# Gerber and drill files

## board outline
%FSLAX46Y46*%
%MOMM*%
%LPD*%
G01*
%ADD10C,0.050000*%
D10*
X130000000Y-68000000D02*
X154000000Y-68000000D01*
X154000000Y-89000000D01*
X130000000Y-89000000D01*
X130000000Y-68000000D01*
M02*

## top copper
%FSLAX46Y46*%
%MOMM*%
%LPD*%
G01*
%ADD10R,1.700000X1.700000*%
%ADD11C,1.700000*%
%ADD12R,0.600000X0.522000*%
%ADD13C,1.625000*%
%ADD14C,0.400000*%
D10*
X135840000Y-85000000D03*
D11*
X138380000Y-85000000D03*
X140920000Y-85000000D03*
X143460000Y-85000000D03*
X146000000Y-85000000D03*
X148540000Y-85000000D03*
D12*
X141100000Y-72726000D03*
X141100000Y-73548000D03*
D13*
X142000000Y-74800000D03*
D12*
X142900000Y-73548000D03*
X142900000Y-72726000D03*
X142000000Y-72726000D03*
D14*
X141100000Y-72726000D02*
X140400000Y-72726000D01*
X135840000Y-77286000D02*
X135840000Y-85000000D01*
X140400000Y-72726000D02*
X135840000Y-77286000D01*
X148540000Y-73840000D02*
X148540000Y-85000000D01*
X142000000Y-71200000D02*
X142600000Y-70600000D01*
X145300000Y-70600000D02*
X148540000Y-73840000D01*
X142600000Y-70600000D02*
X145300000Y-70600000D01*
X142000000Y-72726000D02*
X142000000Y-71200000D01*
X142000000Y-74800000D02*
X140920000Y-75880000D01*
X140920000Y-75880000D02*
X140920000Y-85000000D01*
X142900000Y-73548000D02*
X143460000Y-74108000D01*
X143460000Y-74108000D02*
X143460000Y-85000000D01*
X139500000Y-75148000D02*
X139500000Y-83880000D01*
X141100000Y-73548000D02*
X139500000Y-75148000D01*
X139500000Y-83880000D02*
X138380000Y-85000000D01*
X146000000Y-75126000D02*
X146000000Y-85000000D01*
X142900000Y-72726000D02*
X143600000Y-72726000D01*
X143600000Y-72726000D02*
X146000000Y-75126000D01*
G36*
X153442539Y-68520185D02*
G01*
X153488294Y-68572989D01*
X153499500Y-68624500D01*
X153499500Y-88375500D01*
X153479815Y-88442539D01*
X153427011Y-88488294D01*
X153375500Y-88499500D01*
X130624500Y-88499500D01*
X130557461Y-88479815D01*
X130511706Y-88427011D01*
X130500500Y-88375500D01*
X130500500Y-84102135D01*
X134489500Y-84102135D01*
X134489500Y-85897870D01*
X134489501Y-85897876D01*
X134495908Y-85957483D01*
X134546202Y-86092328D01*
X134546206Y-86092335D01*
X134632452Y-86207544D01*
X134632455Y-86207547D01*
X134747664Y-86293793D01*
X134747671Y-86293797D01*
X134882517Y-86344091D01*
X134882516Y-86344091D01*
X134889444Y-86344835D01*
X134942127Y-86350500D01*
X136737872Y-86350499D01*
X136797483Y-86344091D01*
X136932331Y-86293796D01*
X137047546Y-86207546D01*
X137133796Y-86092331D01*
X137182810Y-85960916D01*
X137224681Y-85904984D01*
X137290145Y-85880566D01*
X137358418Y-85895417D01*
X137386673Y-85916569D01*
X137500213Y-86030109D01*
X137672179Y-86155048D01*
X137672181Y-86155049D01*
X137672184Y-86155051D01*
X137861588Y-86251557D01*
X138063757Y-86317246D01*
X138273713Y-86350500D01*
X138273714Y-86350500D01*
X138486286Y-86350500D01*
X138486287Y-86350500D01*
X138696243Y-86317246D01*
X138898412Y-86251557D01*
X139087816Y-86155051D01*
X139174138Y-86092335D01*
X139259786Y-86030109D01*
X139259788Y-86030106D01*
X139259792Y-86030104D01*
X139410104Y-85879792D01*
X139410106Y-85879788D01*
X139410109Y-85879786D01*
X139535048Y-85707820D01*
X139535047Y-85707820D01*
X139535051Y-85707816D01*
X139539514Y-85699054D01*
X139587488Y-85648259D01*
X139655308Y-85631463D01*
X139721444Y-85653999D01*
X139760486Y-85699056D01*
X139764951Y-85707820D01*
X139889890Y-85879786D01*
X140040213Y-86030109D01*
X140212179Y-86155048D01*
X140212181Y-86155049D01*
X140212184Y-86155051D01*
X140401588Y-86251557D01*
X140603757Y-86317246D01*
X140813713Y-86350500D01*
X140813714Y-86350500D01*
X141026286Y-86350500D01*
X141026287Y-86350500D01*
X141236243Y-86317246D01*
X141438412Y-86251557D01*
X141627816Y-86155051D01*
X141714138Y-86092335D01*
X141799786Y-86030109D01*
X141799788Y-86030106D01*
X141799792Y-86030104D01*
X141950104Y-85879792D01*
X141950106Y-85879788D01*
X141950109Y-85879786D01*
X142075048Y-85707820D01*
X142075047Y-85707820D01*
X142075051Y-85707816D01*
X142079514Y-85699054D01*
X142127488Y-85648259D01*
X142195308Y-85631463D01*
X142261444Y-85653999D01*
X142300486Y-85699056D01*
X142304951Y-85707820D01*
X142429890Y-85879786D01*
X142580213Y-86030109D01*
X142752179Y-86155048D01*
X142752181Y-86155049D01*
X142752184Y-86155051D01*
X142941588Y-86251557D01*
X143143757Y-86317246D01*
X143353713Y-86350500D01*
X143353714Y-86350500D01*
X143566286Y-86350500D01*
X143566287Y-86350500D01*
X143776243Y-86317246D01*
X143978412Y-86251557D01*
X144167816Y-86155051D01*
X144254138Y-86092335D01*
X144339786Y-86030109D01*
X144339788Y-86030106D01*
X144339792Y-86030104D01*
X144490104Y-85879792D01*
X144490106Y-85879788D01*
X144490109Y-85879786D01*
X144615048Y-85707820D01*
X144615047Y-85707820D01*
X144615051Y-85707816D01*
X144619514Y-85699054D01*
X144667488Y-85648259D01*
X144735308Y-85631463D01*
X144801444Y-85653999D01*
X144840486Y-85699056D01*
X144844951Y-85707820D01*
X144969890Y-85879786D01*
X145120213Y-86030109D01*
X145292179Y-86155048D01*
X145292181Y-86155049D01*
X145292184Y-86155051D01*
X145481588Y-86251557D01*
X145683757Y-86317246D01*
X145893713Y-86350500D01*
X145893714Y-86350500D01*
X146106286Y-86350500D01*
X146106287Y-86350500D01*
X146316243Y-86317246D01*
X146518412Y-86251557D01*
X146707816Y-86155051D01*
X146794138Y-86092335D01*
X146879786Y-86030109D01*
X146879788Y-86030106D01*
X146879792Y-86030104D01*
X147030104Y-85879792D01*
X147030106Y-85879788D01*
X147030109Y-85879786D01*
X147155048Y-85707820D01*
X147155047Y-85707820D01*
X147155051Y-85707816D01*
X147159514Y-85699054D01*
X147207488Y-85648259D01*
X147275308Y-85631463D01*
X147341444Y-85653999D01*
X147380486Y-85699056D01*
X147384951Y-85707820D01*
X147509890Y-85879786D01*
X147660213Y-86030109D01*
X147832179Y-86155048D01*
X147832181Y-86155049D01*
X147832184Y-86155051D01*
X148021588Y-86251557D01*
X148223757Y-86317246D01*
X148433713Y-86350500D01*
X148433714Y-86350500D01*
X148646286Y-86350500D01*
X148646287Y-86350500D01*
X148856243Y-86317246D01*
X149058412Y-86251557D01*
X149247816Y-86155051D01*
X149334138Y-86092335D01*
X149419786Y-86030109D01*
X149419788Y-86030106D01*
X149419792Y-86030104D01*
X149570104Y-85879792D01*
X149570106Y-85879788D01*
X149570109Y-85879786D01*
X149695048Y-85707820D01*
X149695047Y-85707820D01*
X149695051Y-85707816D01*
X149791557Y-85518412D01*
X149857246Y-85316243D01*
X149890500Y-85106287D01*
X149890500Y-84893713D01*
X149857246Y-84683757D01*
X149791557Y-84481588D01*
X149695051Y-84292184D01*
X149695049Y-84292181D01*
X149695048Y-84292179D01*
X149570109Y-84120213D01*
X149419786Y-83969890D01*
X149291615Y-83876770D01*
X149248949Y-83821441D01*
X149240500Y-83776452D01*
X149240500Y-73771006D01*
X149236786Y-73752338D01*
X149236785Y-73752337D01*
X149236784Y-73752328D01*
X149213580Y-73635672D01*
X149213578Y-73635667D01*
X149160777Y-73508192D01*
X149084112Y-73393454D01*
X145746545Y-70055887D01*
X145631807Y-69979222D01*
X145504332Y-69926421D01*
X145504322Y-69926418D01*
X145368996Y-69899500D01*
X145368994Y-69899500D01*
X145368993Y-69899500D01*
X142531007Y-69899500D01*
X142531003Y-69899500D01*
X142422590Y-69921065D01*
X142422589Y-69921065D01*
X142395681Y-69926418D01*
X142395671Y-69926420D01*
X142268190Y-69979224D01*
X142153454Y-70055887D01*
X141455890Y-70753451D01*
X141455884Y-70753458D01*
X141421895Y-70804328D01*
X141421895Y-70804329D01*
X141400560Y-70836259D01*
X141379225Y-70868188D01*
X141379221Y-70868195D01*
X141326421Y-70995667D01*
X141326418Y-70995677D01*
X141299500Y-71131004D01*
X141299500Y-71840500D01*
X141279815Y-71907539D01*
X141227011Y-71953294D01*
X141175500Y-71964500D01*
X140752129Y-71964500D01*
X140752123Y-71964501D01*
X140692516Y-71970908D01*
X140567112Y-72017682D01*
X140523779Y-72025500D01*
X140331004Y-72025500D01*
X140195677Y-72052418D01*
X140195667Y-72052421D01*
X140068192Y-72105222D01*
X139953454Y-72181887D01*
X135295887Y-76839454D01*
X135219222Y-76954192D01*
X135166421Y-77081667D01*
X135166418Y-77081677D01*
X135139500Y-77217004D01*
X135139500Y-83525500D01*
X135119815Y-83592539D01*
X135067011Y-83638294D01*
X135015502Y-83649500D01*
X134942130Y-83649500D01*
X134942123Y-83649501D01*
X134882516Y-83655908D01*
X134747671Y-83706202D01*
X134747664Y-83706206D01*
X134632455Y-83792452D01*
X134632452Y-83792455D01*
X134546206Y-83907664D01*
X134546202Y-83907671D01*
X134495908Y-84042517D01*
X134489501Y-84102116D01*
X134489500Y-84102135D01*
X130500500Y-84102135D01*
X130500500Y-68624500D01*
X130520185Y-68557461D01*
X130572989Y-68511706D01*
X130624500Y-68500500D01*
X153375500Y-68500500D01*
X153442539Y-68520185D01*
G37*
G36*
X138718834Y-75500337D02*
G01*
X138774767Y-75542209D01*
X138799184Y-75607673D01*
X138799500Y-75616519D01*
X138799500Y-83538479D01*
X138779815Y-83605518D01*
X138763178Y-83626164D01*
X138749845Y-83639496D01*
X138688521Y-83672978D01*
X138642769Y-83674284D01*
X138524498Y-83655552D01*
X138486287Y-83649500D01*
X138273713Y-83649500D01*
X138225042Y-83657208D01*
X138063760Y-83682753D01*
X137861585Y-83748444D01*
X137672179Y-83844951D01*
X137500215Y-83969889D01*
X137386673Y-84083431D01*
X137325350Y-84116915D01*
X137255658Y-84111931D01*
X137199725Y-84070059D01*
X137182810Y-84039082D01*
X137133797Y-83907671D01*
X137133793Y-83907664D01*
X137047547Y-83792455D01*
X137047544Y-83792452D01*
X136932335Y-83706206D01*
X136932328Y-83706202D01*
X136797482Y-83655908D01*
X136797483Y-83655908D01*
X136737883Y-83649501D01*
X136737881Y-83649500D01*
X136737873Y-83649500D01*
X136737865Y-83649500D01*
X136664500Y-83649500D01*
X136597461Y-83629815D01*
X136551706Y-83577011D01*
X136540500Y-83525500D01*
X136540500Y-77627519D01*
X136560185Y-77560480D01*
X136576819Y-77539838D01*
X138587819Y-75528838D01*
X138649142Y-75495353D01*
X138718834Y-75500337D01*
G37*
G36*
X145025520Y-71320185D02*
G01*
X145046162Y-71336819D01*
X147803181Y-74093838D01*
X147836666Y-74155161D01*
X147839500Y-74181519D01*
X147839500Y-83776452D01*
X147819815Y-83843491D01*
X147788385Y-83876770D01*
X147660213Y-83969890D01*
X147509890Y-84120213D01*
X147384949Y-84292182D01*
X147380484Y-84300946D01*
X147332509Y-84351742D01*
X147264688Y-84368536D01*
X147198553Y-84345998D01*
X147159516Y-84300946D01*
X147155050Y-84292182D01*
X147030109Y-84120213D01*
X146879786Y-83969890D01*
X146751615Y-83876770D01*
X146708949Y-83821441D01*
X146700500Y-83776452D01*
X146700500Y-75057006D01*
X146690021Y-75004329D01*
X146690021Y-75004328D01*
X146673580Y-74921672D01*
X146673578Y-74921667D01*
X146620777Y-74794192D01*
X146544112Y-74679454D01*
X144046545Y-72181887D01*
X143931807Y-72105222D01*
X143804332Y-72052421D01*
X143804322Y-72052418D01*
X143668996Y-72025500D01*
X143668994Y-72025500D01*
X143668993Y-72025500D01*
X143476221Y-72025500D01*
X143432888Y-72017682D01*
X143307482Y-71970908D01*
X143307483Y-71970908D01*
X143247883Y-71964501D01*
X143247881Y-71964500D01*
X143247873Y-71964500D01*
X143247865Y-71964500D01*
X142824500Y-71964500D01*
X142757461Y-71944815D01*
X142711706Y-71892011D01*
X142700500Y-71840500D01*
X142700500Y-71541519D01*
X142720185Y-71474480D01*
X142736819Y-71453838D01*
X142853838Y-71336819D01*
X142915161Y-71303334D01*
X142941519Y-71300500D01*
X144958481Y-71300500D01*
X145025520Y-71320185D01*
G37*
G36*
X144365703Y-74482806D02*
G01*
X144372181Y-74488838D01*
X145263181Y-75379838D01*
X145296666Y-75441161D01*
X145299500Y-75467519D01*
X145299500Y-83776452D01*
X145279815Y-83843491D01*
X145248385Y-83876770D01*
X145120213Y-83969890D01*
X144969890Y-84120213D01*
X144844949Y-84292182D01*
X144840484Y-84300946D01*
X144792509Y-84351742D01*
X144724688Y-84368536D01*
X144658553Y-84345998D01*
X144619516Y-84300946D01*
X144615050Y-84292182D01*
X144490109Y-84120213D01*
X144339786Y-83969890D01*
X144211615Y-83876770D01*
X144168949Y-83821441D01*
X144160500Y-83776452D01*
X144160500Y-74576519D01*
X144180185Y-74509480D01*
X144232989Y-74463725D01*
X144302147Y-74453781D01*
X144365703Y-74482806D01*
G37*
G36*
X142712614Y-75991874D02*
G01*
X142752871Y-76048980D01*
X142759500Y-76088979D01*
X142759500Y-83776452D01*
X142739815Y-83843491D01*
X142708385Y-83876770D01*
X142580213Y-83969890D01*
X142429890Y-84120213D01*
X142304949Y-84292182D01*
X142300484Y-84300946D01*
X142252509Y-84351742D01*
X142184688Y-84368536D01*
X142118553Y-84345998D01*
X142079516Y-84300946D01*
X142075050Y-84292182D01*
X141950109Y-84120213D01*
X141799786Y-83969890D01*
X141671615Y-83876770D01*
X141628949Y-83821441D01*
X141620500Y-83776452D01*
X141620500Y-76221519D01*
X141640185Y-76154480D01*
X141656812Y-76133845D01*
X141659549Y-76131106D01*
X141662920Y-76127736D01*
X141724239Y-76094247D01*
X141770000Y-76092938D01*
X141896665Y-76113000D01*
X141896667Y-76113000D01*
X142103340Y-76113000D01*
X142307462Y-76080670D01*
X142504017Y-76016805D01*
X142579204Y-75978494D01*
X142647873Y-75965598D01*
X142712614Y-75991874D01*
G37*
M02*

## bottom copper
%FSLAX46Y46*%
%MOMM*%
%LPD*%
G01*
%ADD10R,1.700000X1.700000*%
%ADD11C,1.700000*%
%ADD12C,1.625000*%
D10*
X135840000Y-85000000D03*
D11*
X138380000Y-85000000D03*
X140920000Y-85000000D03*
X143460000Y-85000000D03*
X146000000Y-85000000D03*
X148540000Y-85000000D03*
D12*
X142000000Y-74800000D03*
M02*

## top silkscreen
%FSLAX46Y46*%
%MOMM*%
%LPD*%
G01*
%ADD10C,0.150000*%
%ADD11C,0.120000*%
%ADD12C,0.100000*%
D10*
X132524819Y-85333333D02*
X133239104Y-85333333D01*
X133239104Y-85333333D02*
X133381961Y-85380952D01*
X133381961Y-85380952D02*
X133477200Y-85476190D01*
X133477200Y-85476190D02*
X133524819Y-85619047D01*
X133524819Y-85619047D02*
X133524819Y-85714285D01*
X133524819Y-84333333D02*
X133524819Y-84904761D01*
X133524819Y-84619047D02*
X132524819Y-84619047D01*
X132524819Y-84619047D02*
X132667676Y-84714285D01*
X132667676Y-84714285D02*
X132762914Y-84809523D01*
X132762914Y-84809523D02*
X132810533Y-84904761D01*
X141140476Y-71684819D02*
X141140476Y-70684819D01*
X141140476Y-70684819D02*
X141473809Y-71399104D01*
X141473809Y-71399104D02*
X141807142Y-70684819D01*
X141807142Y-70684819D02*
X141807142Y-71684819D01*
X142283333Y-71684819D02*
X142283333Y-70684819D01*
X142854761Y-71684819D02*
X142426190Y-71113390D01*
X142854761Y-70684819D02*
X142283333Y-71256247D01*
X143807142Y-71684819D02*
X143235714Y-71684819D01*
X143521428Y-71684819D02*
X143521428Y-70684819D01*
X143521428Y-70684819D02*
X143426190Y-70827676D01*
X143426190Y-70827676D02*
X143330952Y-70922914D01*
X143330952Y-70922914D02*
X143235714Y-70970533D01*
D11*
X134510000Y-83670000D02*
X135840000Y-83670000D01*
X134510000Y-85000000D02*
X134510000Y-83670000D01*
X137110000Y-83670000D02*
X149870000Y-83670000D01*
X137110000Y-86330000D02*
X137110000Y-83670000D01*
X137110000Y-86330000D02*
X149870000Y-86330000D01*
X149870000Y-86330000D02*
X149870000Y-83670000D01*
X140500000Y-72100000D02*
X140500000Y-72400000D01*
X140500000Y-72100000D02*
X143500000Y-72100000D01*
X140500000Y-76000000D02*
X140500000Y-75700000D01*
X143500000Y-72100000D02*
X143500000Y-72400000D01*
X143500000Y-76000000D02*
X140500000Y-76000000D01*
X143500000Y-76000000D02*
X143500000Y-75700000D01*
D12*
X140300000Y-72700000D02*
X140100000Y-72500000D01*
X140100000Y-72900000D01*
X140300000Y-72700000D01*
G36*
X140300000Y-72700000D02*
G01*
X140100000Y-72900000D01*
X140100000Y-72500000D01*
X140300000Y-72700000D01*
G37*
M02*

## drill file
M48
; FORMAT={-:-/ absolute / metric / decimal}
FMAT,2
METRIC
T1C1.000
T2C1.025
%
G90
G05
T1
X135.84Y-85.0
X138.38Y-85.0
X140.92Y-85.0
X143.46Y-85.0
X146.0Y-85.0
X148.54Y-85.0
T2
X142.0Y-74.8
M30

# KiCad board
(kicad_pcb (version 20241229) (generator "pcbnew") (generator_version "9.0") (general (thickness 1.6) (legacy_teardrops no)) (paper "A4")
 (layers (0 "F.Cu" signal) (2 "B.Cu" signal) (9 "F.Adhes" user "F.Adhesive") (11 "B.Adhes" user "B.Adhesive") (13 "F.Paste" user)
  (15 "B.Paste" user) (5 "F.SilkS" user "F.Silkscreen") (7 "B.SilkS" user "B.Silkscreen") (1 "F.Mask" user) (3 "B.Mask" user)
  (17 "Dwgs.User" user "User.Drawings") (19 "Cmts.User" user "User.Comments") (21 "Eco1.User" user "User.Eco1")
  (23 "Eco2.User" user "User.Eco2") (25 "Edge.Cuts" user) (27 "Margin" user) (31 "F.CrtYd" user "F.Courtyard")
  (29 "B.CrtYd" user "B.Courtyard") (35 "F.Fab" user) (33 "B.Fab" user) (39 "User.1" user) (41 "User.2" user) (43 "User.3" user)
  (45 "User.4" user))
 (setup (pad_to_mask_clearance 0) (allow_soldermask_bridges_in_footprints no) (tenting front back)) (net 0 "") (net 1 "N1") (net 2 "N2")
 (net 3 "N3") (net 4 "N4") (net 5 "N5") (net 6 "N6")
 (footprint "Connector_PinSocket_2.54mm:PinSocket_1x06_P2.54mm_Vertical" (layer "F.Cu") (at 135.84 85 90)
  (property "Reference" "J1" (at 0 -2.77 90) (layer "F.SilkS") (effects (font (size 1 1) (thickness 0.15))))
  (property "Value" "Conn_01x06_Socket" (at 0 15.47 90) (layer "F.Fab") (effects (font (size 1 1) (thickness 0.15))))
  (fp_line (start 1.33 -1.33) (end 1.33 0) (stroke (width 0.12) (type solid)) (layer "F.SilkS"))
  (fp_line (start 0 -1.33) (end 1.33 -1.33) (stroke (width 0.12) (type solid)) (layer "F.SilkS"))
  (fp_line (start 1.33 1.27) (end 1.33 14.03) (stroke (width 0.12) (type solid)) (layer "F.SilkS"))
  (fp_line (start -1.33 1.27) (end 1.33 1.27) (stroke (width 0.12) (type solid)) (layer "F.SilkS"))
  (fp_line (start -1.33 1.27) (end -1.33 14.03) (stroke (width 0.12) (type solid)) (layer "F.SilkS"))
  (fp_line (start -1.33 14.03) (end 1.33 14.03) (stroke (width 0.12) (type solid)) (layer "F.SilkS"))
  (pad "1" thru_hole rect (at 0 0 90) (size 1.7 1.7) (drill 1) (layers "*.Cu" "*.Mask") (remove_unused_layers no) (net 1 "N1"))
  (pad "2" thru_hole circle (at 0 2.54 90) (size 1.7 1.7) (drill 1) (layers "*.Cu" "*.Mask") (remove_unused_layers no) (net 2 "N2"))
  (pad "3" thru_hole circle (at 0 5.08 90) (size 1.7 1.7) (drill 1) (layers "*.Cu" "*.Mask") (remove_unused_layers no) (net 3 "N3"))
  (pad "4" thru_hole circle (at 0 7.62 90) (size 1.7 1.7) (drill 1) (layers "*.Cu" "*.Mask") (remove_unused_layers no) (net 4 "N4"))
  (pad "5" thru_hole circle (at 0 10.16 90) (size 1.7 1.7) (drill 1) (layers "*.Cu" "*.Mask") (remove_unused_layers no) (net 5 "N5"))
  (pad "6" thru_hole circle (at 0 12.7 90) (size 1.7 1.7) (drill 1) (layers "*.Cu" "*.Mask") (remove_unused_layers no) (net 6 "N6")))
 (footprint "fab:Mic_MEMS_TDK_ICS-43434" (layer "F.Cu") (at 142 74)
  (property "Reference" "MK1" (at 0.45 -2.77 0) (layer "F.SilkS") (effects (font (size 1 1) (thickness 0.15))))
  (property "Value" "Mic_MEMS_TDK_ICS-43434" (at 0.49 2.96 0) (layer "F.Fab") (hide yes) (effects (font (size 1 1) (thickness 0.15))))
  (fp_line (start -1.5 -1.9) (end -1.5 -1.6) (stroke (width 0.12) (type solid)) (layer "F.SilkS"))
  (fp_line (start -1.5 -1.9) (end 1.5 -1.9) (stroke (width 0.12) (type solid)) (layer "F.SilkS"))
  (fp_line (start -1.5 2) (end -1.5 1.7) (stroke (width 0.12) (type solid)) (layer "F.SilkS"))
  (fp_line (start 1.5 -1.9) (end 1.5 -1.6) (stroke (width 0.12) (type solid)) (layer "F.SilkS"))
  (fp_line (start 1.5 2) (end -1.5 2) (stroke (width 0.12) (type solid)) (layer "F.SilkS"))
  (fp_line (start 1.5 2) (end 1.5 1.7) (stroke (width 0.12) (type solid)) (layer "F.SilkS"))
  (fp_poly (pts (xy -1.7 -1.3) (xy -1.9 -1.5) (xy -1.9 -1.1)) (stroke (width 0.1) (type solid)) (fill yes) (layer "F.SilkS"))
  (pad "1" smd rect (at -0.9 -1.274) (size 0.6 0.522) (layers "F.Cu" "F.Mask" "F.Paste") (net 1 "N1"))
  (pad "2" smd rect (at -0.9 -0.452) (size 0.6 0.522) (layers "F.Cu" "F.Mask" "F.Paste") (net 2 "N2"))
  (pad "3" thru_hole circle (at 0 0.8) (size 1.625 1.625) (drill 1.025) (layers "*.Cu" "*.Mask") (remove_unused_layers no) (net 3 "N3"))
  (pad "4" smd rect (at 0.9 -0.452) (size 0.6 0.522) (layers "F.Cu" "F.Mask" "F.Paste") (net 4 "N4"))
  (pad "5" smd rect (at 0.9 -1.274) (size 0.6 0.522) (layers "F.Cu" "F.Mask" "F.Paste") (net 5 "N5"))
  (pad "6" smd rect (at 0 -1.274) (size 0.6 0.522) (layers "F.Cu" "F.Mask" "F.Paste") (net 6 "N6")))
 (gr_rect (start 130 68) (end 154 89) (stroke (width 0.05) (type default)) (fill no) (layer "Edge.Cuts"))
 (segment (start 141.1 72.726) (end 140.4 72.726) (width 0.4) (layer "F.Cu") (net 1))
 (segment (start 135.84 77.286) (end 135.84 85) (width 0.4) (layer "F.Cu") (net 1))
 (segment (start 140.4 72.726) (end 135.84 77.286) (width 0.4) (layer "F.Cu") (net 1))
 (segment (start 148.54 73.84) (end 148.54 85) (width 0.4) (layer "F.Cu") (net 6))
 (segment (start 142 71.2) (end 142.6 70.6) (width 0.4) (layer "F.Cu") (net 6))
 (segment (start 145.3 70.6) (end 148.54 73.84) (width 0.4) (layer "F.Cu") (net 6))
 (segment (start 142.6 70.6) (end 145.3 70.6) (width 0.4) (layer "F.Cu") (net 6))
 (segment (start 142 72.726) (end 142 71.2) (width 0.4) (layer "F.Cu") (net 6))
 (segment (start 142 74.8) (end 140.92 75.88) (width 0.4) (layer "F.Cu") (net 3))
 (segment (start 140.92 75.88) (end 140.92 85) (width 0.4) (layer "F.Cu") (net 3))
 (segment (start 142.9 73.548) (end 143.46 74.108) (width 0.4) (layer "F.Cu") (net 4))
 (segment (start 143.46 74.108) (end 143.46 85) (width 0.4) (layer "F.Cu") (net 4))
 (segment (start 139.5 75.148) (end 139.5 83.88) (width 0.4) (layer "F.Cu") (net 2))
 (segment (start 141.1 73.548) (end 139.5 75.148) (width 0.4) (layer "F.Cu") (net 2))
 (segment (start 139.5 83.88) (end 138.38 85) (width 0.4) (layer "F.Cu") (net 2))
 (segment (start 146 75.126) (end 146 85) (width 0.4) (layer "F.Cu") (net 5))
 (segment (start 142.9 72.726) (end 143.6 72.726) (width 0.4) (layer "F.Cu") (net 5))
 (segment (start 143.6 72.726) (end 146 75.126) (width 0.4) (layer "F.Cu") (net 5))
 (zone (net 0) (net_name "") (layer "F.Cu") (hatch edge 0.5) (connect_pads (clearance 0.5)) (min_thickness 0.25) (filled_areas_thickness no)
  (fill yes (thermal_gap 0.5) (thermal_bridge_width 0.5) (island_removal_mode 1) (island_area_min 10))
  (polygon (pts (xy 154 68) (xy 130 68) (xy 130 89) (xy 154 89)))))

